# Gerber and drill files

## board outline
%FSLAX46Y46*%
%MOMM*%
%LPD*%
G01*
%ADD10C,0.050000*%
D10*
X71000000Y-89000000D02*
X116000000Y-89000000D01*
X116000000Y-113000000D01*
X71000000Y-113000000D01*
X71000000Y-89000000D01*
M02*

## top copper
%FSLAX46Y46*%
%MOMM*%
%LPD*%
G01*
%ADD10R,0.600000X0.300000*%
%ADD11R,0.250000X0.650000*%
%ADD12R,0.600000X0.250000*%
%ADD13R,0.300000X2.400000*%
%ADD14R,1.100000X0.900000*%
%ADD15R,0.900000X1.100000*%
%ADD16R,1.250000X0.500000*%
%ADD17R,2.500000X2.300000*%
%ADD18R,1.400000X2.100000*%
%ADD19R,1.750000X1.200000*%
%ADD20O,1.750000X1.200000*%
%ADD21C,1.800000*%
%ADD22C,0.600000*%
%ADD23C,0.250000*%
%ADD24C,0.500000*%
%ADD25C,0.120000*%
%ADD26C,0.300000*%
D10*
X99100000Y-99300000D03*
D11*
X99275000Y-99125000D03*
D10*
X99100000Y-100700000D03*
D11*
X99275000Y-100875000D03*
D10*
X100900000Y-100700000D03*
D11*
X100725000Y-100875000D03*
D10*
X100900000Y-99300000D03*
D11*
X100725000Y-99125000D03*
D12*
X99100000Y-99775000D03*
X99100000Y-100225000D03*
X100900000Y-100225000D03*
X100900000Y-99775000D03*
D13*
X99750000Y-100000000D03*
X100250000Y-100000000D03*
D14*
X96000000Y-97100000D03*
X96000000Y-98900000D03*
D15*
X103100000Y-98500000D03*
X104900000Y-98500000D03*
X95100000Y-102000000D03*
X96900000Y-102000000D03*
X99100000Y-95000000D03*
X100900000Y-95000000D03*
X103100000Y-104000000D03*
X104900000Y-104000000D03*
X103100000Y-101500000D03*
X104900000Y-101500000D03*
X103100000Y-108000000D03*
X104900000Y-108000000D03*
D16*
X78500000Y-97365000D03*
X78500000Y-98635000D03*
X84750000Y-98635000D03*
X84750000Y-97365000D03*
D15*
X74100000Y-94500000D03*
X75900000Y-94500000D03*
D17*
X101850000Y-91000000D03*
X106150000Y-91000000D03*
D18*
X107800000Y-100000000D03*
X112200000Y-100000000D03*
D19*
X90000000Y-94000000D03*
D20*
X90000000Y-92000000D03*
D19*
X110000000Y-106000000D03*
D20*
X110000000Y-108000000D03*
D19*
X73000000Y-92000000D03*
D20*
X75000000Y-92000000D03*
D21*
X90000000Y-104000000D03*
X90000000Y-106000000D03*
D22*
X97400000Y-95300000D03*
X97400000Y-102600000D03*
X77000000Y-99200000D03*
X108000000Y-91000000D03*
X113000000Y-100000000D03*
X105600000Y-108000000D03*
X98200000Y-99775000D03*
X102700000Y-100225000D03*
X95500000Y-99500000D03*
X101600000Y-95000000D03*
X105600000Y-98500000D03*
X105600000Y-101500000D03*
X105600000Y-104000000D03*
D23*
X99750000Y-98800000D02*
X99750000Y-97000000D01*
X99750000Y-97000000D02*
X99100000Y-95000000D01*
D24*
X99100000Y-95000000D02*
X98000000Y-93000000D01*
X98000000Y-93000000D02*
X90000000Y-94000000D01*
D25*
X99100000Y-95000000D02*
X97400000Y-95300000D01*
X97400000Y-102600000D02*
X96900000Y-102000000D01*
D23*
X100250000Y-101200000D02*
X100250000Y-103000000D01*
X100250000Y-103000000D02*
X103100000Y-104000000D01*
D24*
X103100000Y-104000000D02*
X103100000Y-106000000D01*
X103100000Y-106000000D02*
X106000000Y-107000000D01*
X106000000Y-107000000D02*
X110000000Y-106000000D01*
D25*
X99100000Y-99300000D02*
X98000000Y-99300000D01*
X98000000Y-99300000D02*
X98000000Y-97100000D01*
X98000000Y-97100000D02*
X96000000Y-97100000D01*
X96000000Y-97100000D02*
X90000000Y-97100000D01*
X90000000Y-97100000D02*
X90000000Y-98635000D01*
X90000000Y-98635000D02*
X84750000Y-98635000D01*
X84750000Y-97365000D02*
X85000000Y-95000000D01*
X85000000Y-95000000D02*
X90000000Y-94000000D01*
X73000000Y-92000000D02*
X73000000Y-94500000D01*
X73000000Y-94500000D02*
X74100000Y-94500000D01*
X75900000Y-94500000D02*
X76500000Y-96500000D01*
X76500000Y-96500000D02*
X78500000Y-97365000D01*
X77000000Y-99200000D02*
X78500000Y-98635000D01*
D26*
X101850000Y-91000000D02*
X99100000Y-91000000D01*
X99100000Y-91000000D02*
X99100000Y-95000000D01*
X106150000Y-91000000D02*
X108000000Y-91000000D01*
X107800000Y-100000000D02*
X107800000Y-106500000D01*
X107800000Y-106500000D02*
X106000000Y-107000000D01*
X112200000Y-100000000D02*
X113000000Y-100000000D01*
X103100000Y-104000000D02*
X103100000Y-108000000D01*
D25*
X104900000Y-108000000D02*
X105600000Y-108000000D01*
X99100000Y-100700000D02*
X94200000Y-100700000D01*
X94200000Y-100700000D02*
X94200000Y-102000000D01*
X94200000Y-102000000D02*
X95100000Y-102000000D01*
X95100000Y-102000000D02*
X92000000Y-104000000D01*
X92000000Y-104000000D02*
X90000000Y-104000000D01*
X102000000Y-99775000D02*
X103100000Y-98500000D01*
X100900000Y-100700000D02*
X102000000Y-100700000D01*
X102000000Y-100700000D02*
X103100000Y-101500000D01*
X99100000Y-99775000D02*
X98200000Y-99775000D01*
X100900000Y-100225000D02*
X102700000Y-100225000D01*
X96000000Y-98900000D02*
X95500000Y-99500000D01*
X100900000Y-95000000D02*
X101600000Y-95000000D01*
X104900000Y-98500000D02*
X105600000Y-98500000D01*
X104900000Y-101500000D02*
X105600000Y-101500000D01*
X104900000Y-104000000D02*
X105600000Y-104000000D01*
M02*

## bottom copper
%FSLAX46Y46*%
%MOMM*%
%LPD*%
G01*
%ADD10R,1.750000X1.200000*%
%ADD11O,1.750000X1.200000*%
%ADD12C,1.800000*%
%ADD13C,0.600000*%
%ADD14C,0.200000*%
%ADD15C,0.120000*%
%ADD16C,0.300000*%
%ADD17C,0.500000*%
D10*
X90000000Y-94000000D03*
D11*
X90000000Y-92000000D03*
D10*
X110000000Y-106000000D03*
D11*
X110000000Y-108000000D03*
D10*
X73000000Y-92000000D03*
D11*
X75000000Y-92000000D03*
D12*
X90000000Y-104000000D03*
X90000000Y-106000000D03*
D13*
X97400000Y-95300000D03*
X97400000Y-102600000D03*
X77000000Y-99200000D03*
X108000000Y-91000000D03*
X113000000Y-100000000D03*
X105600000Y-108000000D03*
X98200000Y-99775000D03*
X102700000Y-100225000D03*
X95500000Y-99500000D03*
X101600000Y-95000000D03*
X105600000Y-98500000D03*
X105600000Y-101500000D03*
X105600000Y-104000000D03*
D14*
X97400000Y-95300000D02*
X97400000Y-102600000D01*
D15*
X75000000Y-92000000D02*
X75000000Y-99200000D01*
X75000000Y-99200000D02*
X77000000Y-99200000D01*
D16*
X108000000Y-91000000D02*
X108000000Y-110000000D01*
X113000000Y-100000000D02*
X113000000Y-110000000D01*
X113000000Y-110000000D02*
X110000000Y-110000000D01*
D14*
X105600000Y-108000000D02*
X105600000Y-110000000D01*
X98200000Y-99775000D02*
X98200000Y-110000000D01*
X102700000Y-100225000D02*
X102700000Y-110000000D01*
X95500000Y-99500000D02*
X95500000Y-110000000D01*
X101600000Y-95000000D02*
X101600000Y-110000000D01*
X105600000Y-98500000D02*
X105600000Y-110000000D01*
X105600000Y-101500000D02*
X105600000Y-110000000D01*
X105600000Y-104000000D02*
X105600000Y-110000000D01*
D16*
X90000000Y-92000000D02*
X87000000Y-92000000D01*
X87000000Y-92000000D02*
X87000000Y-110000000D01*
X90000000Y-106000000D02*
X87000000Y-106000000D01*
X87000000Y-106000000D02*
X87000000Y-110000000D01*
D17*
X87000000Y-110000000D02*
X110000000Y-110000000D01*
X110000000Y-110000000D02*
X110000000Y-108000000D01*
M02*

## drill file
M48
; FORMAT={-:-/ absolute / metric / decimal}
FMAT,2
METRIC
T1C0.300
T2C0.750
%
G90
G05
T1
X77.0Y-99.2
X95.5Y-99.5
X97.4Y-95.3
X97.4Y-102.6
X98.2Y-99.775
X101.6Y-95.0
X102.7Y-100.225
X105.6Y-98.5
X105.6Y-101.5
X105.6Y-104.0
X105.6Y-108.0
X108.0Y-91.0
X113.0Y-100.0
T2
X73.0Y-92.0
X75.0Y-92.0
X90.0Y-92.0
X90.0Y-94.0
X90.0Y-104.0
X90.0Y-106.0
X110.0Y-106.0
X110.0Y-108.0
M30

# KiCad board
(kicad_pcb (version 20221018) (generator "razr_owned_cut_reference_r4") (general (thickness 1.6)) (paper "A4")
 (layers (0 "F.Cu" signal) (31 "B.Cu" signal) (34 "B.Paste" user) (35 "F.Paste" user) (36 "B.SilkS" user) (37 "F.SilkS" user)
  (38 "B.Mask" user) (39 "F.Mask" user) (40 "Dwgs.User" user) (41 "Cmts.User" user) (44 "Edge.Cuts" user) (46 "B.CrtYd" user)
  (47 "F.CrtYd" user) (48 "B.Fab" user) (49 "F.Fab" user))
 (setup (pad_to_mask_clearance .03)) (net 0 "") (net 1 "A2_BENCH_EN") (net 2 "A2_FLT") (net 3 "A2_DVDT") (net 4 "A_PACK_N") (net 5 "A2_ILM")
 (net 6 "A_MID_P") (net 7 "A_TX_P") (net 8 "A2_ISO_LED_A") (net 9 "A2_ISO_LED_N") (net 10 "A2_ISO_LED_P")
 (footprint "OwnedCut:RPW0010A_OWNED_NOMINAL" (layer "F.Cu") (at 100 100)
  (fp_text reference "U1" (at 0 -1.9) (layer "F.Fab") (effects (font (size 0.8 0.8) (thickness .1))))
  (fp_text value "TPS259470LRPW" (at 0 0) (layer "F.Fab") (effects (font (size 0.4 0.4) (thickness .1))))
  (pad "1" smd rect (at -0.9 -0.7) (size 0.6 0.3) (layers "F.Cu" "F.Paste" "F.Mask") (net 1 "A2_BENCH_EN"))
  (pad "1" smd rect (at -0.725 -0.875) (size 0.25 0.65) (layers "F.Cu" "F.Paste" "F.Mask") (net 1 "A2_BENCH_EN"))
  (pad "4" smd rect (at -0.9 0.7) (size 0.6 0.3) (layers "F.Cu" "F.Paste" "F.Mask") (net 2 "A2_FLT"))
  (pad "4" smd rect (at -0.725 0.875) (size 0.25 0.65) (layers "F.Cu" "F.Paste" "F.Mask") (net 2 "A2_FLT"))
  (pad "7" smd rect (at 0.9 0.7) (size 0.6 0.3) (layers "F.Cu" "F.Paste" "F.Mask") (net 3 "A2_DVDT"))
  (pad "7" smd rect (at 0.725 0.875) (size 0.25 0.65) (layers "F.Cu" "F.Paste" "F.Mask") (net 3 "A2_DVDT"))
  (pad "10" smd rect (at 0.9 -0.7) (size 0.6 0.3) (layers "F.Cu" "F.Paste" "F.Mask"))
  (pad "10" smd rect (at 0.725 -0.875) (size 0.25 0.65) (layers "F.Cu" "F.Paste" "F.Mask"))
  (pad "2" smd rect (at -0.9 -0.225) (size 0.6 0.25) (layers "F.Cu" "F.Paste" "F.Mask") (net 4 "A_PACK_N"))
  (pad "3" smd rect (at -0.9 0.225) (size 0.6 0.25) (layers "F.Cu" "F.Paste" "F.Mask"))
  (pad "8" smd rect (at 0.9 0.225) (size 0.6 0.25) (layers "F.Cu" "F.Paste" "F.Mask") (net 4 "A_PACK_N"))
  (pad "9" smd rect (at 0.9 -0.225) (size 0.6 0.25) (layers "F.Cu" "F.Paste" "F.Mask") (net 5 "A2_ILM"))
  (pad "5" smd rect (at -0.25 0) (size 0.3 2.4) (layers "F.Cu" "F.Paste" "F.Mask") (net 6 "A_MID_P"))
  (pad "6" smd rect (at 0.25 0) (size 0.3 2.4) (layers "F.Cu" "F.Paste" "F.Mask") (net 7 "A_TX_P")))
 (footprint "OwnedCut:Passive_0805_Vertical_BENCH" (layer "F.Cu") (at 96 98)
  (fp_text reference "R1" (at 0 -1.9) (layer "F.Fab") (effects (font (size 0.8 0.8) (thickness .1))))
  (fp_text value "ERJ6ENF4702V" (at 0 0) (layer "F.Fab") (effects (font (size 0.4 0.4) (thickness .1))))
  (pad "1" smd rect (at 0 -0.9) (size 1.1 0.9) (layers "F.Cu" "F.Paste" "F.Mask") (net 1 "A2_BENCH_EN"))
  (pad "2" smd rect (at 0 0.9) (size 1.1 0.9) (layers "F.Cu" "F.Paste" "F.Mask") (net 4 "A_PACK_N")))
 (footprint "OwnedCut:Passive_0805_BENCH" (layer "F.Cu") (at 104 98.5)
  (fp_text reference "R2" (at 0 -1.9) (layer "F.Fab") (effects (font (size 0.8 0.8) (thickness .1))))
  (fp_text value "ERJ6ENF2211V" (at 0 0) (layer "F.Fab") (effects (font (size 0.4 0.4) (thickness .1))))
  (pad "1" smd rect (at -0.9 0) (size 0.9 1.1) (layers "F.Cu" "F.Paste" "F.Mask") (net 5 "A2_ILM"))
  (pad "2" smd rect (at 0.9 0) (size 0.9 1.1) (layers "F.Cu" "F.Paste" "F.Mask") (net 4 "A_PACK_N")))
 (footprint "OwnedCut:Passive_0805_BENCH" (layer "F.Cu") (at 96 102)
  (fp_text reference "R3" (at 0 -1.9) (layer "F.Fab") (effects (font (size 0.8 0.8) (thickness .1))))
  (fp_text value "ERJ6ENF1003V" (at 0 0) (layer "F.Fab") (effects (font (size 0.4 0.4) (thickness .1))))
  (pad "1" smd rect (at -0.9 0) (size 0.9 1.1) (layers "F.Cu" "F.Paste" "F.Mask") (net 2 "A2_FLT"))
  (pad "2" smd rect (at 0.9 0) (size 0.9 1.1) (layers "F.Cu" "F.Paste" "F.Mask") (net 6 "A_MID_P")))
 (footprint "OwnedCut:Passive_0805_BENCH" (layer "F.Cu") (at 100 95)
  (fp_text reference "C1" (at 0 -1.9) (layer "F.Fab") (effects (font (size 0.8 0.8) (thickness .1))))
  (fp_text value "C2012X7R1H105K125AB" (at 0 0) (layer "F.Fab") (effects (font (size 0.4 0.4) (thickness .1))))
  (pad "1" smd rect (at -0.9 0) (size 0.9 1.1) (layers "F.Cu" "F.Paste" "F.Mask") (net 6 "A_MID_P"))
  (pad "2" smd rect (at 0.9 0) (size 0.9 1.1) (layers "F.Cu" "F.Paste" "F.Mask") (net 4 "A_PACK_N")))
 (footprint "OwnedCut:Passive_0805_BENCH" (layer "F.Cu") (at 104 104)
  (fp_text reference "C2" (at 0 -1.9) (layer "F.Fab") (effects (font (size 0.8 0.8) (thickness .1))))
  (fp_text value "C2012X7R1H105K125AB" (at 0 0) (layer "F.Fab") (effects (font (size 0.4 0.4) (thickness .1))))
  (pad "1" smd rect (at -0.9 0) (size 0.9 1.1) (layers "F.Cu" "F.Paste" "F.Mask") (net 7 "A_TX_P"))
  (pad "2" smd rect (at 0.9 0) (size 0.9 1.1) (layers "F.Cu" "F.Paste" "F.Mask") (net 4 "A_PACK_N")))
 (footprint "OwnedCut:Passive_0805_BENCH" (layer "F.Cu") (at 104 101.5)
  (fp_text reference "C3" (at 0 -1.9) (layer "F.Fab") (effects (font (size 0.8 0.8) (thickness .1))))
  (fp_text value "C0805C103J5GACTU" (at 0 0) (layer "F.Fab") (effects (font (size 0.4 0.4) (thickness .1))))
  (pad "1" smd rect (at -0.9 0) (size 0.9 1.1) (layers "F.Cu" "F.Paste" "F.Mask") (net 3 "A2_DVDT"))
  (pad "2" smd rect (at 0.9 0) (size 0.9 1.1) (layers "F.Cu" "F.Paste" "F.Mask") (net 4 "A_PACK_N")))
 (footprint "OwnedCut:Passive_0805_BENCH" (layer "F.Cu") (at 104 108)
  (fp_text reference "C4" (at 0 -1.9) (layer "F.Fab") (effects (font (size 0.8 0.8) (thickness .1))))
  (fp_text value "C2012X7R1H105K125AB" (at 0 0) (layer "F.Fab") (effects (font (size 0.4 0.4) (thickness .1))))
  (pad "1" smd rect (at -0.9 0) (size 0.9 1.1) (layers "F.Cu" "F.Paste" "F.Mask") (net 7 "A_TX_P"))
  (pad "2" smd rect (at 0.9 0) (size 0.9 1.1) (layers "F.Cu" "F.Paste" "F.Mask") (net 4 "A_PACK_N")))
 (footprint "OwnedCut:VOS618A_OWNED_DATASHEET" (layer "F.Cu") (at 81.625 98)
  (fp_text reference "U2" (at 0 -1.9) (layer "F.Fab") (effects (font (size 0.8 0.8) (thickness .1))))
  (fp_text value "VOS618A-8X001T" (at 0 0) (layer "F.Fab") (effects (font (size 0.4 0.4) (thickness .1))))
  (pad "1" smd rect (at -3.125 -0.635) (size 1.25 0.5) (layers "F.Cu" "F.Paste" "F.Mask") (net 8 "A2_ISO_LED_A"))
  (pad "2" smd rect (at -3.125 0.635) (size 1.25 0.5) (layers "F.Cu" "F.Paste" "F.Mask") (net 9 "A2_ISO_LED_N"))
  (pad "3" smd rect (at 3.125 0.635) (size 1.25 0.5) (layers "F.Cu" "F.Paste" "F.Mask") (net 1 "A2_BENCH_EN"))
  (pad "4" smd rect (at 3.125 -0.635) (size 1.25 0.5) (layers "F.Cu" "F.Paste" "F.Mask") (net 6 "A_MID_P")))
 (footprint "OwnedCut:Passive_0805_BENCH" (layer "F.Cu") (at 75 94.5)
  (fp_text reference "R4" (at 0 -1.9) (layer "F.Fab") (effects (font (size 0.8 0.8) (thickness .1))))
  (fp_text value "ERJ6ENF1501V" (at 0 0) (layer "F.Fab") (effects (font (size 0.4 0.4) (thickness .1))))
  (pad "1" smd rect (at -0.9 0) (size 0.9 1.1) (layers "F.Cu" "F.Paste" "F.Mask") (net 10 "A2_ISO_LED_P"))
  (pad "2" smd rect (at 0.9 0) (size 0.9 1.1) (layers "F.Cu" "F.Paste" "F.Mask") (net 8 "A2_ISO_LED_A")))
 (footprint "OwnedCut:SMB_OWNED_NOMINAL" (layer "F.Cu") (at 104 91)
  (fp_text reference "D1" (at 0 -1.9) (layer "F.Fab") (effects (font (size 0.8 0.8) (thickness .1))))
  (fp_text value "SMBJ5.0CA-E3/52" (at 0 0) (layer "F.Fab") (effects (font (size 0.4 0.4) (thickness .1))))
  (pad "1" smd rect (at -2.15 0) (size 2.5 2.3) (layers "F.Cu" "F.Paste" "F.Mask") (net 6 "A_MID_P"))
  (pad "2" smd rect (at 2.15 0) (size 2.5 2.3) (layers "F.Cu" "F.Paste" "F.Mask") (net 4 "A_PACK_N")))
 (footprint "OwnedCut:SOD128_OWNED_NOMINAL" (layer "F.Cu") (at 110 100)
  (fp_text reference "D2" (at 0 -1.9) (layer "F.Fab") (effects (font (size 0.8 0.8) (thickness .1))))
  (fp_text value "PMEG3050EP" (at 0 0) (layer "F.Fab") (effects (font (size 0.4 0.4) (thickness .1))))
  (pad "1" smd rect (at -2.2 0) (size 1.4 2.1) (layers "F.Cu" "F.Paste" "F.Mask") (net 7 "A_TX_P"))
  (pad "2" smd rect (at 2.2 0) (size 1.4 2.1) (layers "F.Cu" "F.Paste" "F.Mask") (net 4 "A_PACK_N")))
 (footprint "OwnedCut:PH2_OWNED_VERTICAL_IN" (layer "F.Cu") (at 90 94)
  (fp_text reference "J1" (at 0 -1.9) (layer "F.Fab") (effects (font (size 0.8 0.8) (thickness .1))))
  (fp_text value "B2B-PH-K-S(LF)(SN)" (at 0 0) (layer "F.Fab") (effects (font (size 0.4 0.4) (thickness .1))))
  (pad "1" thru_hole rect (at 0 0) (size 1.75 1.2) (drill .75) (layers "*.Cu" "*.Mask") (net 6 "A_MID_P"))
  (pad "2" thru_hole oval (at 0 -2) (size 1.75 1.2) (drill .75) (layers "*.Cu" "*.Mask") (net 4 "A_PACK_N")))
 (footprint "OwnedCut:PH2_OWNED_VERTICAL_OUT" (layer "F.Cu") (at 110 106)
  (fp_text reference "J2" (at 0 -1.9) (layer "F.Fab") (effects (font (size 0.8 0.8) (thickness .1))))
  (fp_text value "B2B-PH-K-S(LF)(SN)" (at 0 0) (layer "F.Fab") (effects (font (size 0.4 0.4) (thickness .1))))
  (pad "1" thru_hole rect (at 0 0) (size 1.75 1.2) (drill .75) (layers "*.Cu" "*.Mask") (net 7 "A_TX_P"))
  (pad "2" thru_hole oval (at 0 2) (size 1.75 1.2) (drill .75) (layers "*.Cu" "*.Mask") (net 4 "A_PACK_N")))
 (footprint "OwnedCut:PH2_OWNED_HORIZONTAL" (layer "F.Cu") (at 73 92)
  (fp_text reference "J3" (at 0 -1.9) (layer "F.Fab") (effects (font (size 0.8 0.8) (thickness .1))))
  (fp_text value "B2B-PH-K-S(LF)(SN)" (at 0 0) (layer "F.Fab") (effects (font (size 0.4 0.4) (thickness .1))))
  (pad "1" thru_hole rect (at 0 0) (size 1.75 1.2) (drill .75) (layers "*.Cu" "*.Mask") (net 10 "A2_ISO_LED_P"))
  (pad "2" thru_hole oval (at 2 0) (size 1.75 1.2) (drill .75) (layers "*.Cu" "*.Mask") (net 9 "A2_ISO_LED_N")))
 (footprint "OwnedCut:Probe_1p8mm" (layer "F.Cu") (at 90 104)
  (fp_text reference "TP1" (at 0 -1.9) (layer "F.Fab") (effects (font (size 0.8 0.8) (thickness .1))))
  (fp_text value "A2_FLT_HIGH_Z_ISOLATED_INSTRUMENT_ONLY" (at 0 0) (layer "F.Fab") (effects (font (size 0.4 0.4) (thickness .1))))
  (pad "1" thru_hole circle (at 0 0) (size 1.8 1.8) (drill .75) (layers "*.Cu" "*.Mask") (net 2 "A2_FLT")))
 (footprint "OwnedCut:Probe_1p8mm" (layer "F.Cu") (at 90 106)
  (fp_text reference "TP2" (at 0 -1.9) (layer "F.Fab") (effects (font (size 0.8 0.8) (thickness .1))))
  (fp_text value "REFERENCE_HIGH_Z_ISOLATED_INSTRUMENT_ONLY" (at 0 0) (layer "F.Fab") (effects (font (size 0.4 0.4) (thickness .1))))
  (pad "1" thru_hole circle (at 0 0) (size 1.8 1.8) (drill .75) (layers "*.Cu" "*.Mask") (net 4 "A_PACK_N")))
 (segment (start 99.75 98.8) (end 99.75 97) (width 0.25) (layer "F.Cu") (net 6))
 (segment (start 99.75 97) (end 99.1 95) (width 0.25) (layer "F.Cu") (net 6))
 (segment (start 99.1 95) (end 98 93) (width 0.5) (layer "F.Cu") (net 6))
 (segment (start 98 93) (end 90 94) (width 0.5) (layer "F.Cu") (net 6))
 (segment (start 99.1 95) (end 97.4 95.3) (width 0.12) (layer "F.Cu") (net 6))
 (via (at 97.4 95.3) (size .6) (drill .3) (layers "F.Cu" "B.Cu") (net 6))
 (segment (start 97.4 95.3) (end 97.4 102.6) (width 0.2) (layer "B.Cu") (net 6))
 (via (at 97.4 102.6) (size .6) (drill .3) (layers "F.Cu" "B.Cu") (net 6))
 (segment (start 97.4 102.6) (end 96.9 102) (width 0.12) (layer "F.Cu") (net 6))
 (segment (start 100.25 101.2) (end 100.25 103) (width 0.25) (layer "F.Cu") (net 7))
 (segment (start 100.25 103) (end 103.1 104) (width 0.25) (layer "F.Cu") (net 7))
 (segment (start 103.1 104) (end 103.1 106) (width 0.5) (layer "F.Cu") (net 7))
 (segment (start 103.1 106) (end 106 107) (width 0.5) (layer "F.Cu") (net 7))
 (segment (start 106 107) (end 110 106) (width 0.5) (layer "F.Cu") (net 7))
 (segment (start 99.1 99.3) (end 98 99.3) (width 0.12) (layer "F.Cu") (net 1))
 (segment (start 98 99.3) (end 98 97.1) (width 0.12) (layer "F.Cu") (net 1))
 (segment (start 98 97.1) (end 96 97.1) (width 0.12) (layer "F.Cu") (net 1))
 (segment (start 96 97.1) (end 90 97.1) (width 0.12) (layer "F.Cu") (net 1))
 (segment (start 90 97.1) (end 90 98.635) (width 0.12) (layer "F.Cu") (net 1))
 (segment (start 90 98.635) (end 84.75 98.635) (width 0.12) (layer "F.Cu") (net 1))
 (segment (start 84.75 97.365) (end 85 95) (width 0.12) (layer "F.Cu") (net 6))
 (segment (start 85 95) (end 90 94) (width 0.12) (layer "F.Cu") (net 6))
 (segment (start 73 92) (end 73 94.5) (width 0.12) (layer "F.Cu") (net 10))
 (segment (start 73 94.5) (end 74.1 94.5) (width 0.12) (layer "F.Cu") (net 10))
 (segment (start 75.9 94.5) (end 76.5 96.5) (width 0.12) (layer "F.Cu") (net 8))
 (segment (start 76.5 96.5) (end 78.5 97.365) (width 0.12) (layer "F.Cu") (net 8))
 (segment (start 75 92) (end 75 99.2) (width 0.12) (layer "B.Cu") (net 9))
 (segment (start 75 99.2) (end 77 99.2) (width 0.12) (layer "B.Cu") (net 9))
 (via (at 77 99.2) (size .6) (drill .3) (layers "F.Cu" "B.Cu") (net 9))
 (segment (start 77 99.2) (end 78.5 98.635) (width 0.12) (layer "F.Cu") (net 9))
 (segment (start 101.85 91) (end 99.1 91) (width 0.3) (layer "F.Cu") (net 6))
 (segment (start 99.1 91) (end 99.1 95) (width 0.3) (layer "F.Cu") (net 6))
 (segment (start 106.15 91) (end 108 91) (width 0.3) (layer "F.Cu") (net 4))
 (via (at 108 91) (size .6) (drill .3) (layers "F.Cu" "B.Cu") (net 4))
 (segment (start 108 91) (end 108 110) (width 0.3) (layer "B.Cu") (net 4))
 (segment (start 107.8 100) (end 107.8 106.5) (width 0.3) (layer "F.Cu") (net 7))
 (segment (start 107.8 106.5) (end 106 107) (width 0.3) (layer "F.Cu") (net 7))
 (segment (start 112.2 100) (end 113 100) (width 0.3) (layer "F.Cu") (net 4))
 (via (at 113 100) (size .6) (drill .3) (layers "F.Cu" "B.Cu") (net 4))
 (segment (start 113 100) (end 113 110) (width 0.3) (layer "B.Cu") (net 4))
 (segment (start 113 110) (end 110 110) (width 0.3) (layer "B.Cu") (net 4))
 (segment (start 103.1 104) (end 103.1 108) (width 0.3) (layer "F.Cu") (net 7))
 (segment (start 104.9 108) (end 105.6 108) (width 0.12) (layer "F.Cu") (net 4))
 (via (at 105.6 108) (size .6) (drill .3) (layers "F.Cu" "B.Cu") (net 4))
 (segment (start 105.6 108) (end 105.6 110) (width 0.2) (layer "B.Cu") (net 4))
 (segment (start 99.1 100.7) (end 94.2 100.7) (width 0.12) (layer "F.Cu") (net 2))
 (segment (start 94.2 100.7) (end 94.2 102) (width 0.12) (layer "F.Cu") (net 2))
 (segment (start 94.2 102) (end 95.1 102) (width 0.12) (layer "F.Cu") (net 2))
 (segment (start 95.1 102) (end 92 104) (width 0.12) (layer "F.Cu") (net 2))
 (segment (start 92 104) (end 90 104) (width 0.12) (layer "F.Cu") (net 2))
 (segment (start 102 99.775) (end 103.1 98.5) (width 0.12) (layer "F.Cu") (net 5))
 (segment (start 100.9 100.7) (end 102 100.7) (width 0.12) (layer "F.Cu") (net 3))
 (segment (start 102 100.7) (end 103.1 101.5) (width 0.12) (layer "F.Cu") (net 3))
 (segment (start 99.1 99.775) (end 98.2 99.775) (width 0.12) (layer "F.Cu") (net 4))
 (via (at 98.2 99.775) (size .6) (drill .3) (layers "F.Cu" "B.Cu") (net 4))
 (segment (start 98.2 99.775) (end 98.2 110) (width 0.2) (layer "B.Cu") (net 4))
 (segment (start 100.9 100.225) (end 102.7 100.225) (width 0.12) (layer "F.Cu") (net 4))
 (via (at 102.7 100.225) (size .6) (drill .3) (layers "F.Cu" "B.Cu") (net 4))
 (segment (start 102.7 100.225) (end 102.7 110) (width 0.2) (layer "B.Cu") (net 4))
 (segment (start 96 98.9) (end 95.5 99.5) (width 0.12) (layer "F.Cu") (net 4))
 (via (at 95.5 99.5) (size .6) (drill .3) (layers "F.Cu" "B.Cu") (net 4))
 (segment (start 95.5 99.5) (end 95.5 110) (width 0.2) (layer "B.Cu") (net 4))
 (segment (start 100.9 95) (end 101.6 95) (width 0.12) (layer "F.Cu") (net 4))
 (via (at 101.6 95) (size .6) (drill .3) (layers "F.Cu" "B.Cu") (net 4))
 (segment (start 101.6 95) (end 101.6 110) (width 0.2) (layer "B.Cu") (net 4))
 (segment (start 104.9 98.5) (end 105.6 98.5) (width 0.12) (layer "F.Cu") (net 4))
 (via (at 105.6 98.5) (size .6) (drill .3) (layers "F.Cu" "B.Cu") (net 4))
 (segment (start 105.6 98.5) (end 105.6 110) (width 0.2) (layer "B.Cu") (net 4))
 (segment (start 104.9 101.5) (end 105.6 101.5) (width 0.12) (layer "F.Cu") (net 4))
 (via (at 105.6 101.5) (size .6) (drill .3) (layers "F.Cu" "B.Cu") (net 4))
 (segment (start 105.6 101.5) (end 105.6 110) (width 0.2) (layer "B.Cu") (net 4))
 (segment (start 104.9 104) (end 105.6 104) (width 0.12) (layer "F.Cu") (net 4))
 (via (at 105.6 104) (size .6) (drill .3) (layers "F.Cu" "B.Cu") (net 4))
 (segment (start 105.6 104) (end 105.6 110) (width 0.2) (layer "B.Cu") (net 4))
 (segment (start 90 92) (end 87 92) (width 0.3) (layer "B.Cu") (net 4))
 (segment (start 87 92) (end 87 110) (width 0.3) (layer "B.Cu") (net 4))
 (segment (start 90 106) (end 87 106) (width 0.3) (layer "B.Cu") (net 4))
 (segment (start 87 106) (end 87 110) (width 0.3) (layer "B.Cu") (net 4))
 (segment (start 87 110) (end 110 110) (width 0.5) (layer "B.Cu") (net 4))
 (segment (start 110 110) (end 110 108) (width 0.5) (layer "B.Cu") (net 4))
 (gr_rect (start 71 89) (end 116 113) (stroke (width .05) (type default)) (fill none) (layer "Edge.Cuts")))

